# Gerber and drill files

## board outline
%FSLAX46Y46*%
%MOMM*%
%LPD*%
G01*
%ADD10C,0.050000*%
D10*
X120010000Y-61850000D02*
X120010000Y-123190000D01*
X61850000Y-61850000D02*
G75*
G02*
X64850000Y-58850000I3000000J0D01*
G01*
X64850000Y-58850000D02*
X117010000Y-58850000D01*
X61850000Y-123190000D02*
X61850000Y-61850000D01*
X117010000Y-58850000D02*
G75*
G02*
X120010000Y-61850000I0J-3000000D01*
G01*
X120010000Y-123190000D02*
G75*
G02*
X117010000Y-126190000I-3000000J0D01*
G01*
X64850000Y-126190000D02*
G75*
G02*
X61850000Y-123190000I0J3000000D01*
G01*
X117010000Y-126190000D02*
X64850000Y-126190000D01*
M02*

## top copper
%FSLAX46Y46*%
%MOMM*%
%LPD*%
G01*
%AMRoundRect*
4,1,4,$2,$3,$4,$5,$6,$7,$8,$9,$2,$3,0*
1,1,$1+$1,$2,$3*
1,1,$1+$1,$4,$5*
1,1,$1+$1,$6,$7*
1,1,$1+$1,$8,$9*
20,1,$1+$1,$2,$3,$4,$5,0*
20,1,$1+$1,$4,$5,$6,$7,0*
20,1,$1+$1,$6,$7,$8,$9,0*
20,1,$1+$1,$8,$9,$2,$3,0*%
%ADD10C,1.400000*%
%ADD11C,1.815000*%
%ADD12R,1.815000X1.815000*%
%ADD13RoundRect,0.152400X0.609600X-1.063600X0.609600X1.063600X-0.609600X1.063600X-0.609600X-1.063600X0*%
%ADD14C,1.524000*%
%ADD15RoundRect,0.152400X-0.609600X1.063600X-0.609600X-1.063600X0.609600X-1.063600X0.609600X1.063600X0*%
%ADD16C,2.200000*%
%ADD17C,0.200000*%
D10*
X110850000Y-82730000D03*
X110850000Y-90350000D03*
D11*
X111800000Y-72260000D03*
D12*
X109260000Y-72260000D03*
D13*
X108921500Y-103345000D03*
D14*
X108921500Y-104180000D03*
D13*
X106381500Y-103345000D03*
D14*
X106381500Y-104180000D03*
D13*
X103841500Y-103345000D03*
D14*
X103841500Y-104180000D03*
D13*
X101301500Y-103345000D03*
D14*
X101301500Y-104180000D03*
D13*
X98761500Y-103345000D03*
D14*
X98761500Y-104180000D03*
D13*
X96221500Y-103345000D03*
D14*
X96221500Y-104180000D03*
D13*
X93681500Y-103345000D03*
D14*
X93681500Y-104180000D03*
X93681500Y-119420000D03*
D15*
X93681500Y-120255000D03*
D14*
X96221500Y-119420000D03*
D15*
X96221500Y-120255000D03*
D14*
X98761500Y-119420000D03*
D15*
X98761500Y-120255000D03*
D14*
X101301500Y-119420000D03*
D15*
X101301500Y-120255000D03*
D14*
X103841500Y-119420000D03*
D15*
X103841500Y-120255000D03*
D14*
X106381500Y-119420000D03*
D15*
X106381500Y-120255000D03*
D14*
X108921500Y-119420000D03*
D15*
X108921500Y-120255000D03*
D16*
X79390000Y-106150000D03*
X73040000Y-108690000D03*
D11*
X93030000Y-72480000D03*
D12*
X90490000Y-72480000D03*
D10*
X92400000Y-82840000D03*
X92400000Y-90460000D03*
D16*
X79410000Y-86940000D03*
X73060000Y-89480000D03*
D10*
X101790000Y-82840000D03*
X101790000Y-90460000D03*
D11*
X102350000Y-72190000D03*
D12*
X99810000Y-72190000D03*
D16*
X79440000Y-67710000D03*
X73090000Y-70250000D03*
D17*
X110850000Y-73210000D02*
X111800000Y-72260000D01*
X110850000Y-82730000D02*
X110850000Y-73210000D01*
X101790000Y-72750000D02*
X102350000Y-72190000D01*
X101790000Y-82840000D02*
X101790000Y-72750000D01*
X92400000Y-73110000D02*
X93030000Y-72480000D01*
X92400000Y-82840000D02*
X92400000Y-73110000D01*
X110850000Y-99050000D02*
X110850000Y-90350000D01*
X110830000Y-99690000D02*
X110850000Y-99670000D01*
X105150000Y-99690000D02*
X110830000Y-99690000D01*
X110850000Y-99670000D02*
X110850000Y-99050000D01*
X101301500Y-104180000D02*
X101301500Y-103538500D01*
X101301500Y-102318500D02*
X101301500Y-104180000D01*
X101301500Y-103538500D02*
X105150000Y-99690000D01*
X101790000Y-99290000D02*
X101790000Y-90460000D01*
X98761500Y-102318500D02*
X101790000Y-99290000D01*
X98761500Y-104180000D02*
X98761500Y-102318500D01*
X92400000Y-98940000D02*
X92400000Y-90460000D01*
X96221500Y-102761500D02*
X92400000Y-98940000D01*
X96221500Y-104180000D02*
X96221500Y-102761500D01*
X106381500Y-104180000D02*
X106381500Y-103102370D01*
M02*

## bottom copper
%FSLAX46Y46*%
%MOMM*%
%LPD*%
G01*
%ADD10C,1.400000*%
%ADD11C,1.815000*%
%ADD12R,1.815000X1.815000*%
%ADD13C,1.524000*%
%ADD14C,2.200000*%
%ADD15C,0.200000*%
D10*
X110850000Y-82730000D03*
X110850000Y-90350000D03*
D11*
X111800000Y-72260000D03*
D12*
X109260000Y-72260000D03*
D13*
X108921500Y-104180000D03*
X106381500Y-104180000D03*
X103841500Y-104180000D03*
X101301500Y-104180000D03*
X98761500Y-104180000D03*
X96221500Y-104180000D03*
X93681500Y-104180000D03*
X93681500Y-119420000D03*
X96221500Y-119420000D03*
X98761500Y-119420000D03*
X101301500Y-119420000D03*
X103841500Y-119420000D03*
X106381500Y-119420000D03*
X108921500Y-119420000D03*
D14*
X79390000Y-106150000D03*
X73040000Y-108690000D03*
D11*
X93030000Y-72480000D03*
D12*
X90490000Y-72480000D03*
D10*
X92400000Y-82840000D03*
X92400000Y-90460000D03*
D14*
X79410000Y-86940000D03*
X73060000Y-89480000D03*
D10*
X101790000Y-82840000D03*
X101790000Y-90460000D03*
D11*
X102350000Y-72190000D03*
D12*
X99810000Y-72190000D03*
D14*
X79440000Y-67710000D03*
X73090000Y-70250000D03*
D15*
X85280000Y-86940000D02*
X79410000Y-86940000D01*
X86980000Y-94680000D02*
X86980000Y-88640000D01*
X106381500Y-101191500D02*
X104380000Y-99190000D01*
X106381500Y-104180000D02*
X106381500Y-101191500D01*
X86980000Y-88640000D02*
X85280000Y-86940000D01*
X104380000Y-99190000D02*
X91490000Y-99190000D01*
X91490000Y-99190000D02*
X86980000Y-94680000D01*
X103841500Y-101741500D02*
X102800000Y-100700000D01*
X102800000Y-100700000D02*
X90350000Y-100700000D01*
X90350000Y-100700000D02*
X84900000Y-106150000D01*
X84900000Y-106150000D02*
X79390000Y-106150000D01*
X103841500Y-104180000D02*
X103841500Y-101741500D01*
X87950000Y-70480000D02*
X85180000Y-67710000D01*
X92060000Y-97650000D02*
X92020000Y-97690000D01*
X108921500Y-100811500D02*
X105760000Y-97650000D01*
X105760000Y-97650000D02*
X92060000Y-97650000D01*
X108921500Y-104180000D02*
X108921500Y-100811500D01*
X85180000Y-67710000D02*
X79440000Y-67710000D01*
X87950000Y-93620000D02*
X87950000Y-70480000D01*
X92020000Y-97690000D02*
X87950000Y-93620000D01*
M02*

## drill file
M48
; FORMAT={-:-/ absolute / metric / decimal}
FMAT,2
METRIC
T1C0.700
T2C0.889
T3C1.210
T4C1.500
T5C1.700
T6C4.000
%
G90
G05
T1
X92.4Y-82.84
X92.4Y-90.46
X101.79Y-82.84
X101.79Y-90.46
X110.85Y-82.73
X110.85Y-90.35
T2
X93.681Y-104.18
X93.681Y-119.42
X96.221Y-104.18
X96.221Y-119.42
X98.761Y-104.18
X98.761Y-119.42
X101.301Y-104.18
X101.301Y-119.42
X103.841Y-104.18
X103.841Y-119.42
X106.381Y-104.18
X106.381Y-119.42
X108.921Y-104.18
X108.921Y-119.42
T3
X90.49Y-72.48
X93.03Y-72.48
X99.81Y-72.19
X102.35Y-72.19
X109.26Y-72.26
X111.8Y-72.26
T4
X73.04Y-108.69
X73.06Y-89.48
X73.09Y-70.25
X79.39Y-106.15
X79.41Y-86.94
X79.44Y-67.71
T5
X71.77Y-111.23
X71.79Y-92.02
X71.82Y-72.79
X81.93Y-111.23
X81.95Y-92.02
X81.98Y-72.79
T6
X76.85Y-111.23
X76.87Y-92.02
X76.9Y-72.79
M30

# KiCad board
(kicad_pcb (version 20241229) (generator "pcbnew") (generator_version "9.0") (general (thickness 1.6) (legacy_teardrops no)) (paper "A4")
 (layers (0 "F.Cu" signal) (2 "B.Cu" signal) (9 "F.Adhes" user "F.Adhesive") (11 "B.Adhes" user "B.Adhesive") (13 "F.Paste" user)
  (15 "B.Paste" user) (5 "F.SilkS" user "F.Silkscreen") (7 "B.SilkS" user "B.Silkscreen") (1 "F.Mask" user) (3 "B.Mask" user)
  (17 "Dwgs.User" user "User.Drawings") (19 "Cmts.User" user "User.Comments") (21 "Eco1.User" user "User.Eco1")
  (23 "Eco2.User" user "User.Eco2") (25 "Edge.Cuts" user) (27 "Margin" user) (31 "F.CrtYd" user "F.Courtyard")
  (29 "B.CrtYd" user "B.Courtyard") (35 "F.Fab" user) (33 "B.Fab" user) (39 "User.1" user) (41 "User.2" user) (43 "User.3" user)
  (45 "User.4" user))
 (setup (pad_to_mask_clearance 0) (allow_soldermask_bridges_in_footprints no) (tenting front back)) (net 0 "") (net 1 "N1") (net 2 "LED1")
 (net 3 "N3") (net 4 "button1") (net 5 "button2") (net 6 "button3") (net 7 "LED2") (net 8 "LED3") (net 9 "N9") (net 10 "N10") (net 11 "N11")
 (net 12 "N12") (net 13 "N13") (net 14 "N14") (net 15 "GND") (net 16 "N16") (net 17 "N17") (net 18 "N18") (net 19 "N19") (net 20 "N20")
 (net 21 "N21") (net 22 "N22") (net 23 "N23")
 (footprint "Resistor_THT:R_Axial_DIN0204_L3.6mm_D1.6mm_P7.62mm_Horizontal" (layer "F.Cu") (at 110.85 82.73 -90)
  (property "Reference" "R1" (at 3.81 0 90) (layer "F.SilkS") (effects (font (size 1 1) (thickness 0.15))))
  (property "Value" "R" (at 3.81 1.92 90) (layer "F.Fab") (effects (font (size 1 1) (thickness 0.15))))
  (pad "1" thru_hole circle (at 0 0 270) (size 1.4 1.4) (drill 0.7) (layers "*.Cu" "*.Mask") (remove_unused_layers no) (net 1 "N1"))
  (pad "2" thru_hole circle (at 7.62 0 270) (size 1.4 1.4) (drill 0.7) (layers "*.Cu" "*.Mask") (remove_unused_layers no) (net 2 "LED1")))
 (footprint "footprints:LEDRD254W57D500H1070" (layer "F.Cu") (at 110.53 72.26)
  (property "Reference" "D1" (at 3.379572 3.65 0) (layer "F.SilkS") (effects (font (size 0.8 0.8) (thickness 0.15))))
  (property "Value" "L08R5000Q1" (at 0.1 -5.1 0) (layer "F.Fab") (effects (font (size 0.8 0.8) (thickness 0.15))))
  (pad "A" thru_hole circle (at 1.27 0) (size 1.815 1.815) (drill 1.21) (layers "*.Cu" "*.Mask") (remove_unused_layers no) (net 1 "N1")
   (solder_mask_margin 0.102))
  (pad "C" thru_hole rect (at -1.27 0) (size 1.815 1.815) (drill 1.21) (layers "*.Cu" "*.Mask") (remove_unused_layers no) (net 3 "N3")
   (solder_mask_margin 0.102)))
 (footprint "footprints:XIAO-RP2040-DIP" (layer "F.Cu") (at 101.3015 111.8 -90)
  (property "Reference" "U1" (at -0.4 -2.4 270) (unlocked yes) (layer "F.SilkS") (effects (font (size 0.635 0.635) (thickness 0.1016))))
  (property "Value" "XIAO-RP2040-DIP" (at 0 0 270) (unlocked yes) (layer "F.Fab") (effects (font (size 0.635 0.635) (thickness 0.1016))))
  (pad "1" smd roundrect (at -8.455 -7.62 90) (size 2.432 1.524) (layers "F.Cu" "F.Mask") (roundrect_rratio 0.1) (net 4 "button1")
   (thermal_bridge_angle 45))
  (pad "1" thru_hole circle (at -7.62 -7.62 90) (size 1.524 1.524) (drill 0.889) (layers "*.Cu" "*.Mask") (remove_unused_layers no)
   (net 4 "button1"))
  (pad "2" smd roundrect (at -8.455 -5.08 90) (size 2.432 1.524) (layers "F.Cu" "F.Mask") (roundrect_rratio 0.1) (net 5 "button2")
   (thermal_bridge_angle 45))
  (pad "2" thru_hole circle (at -7.62 -5.08 90) (size 1.524 1.524) (drill 0.889) (layers "*.Cu" "*.Mask") (remove_unused_layers no)
   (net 5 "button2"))
  (pad "3" smd roundrect (at -8.455 -2.54 90) (size 2.432 1.524) (layers "F.Cu" "F.Mask") (roundrect_rratio 0.1) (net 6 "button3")
   (thermal_bridge_angle 45))
  (pad "3" thru_hole circle (at -7.62 -2.54 90) (size 1.524 1.524) (drill 0.889) (layers "*.Cu" "*.Mask") (remove_unused_layers no)
   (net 6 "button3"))
  (pad "4" smd roundrect (at -8.455 0 90) (size 2.432 1.524) (layers "F.Cu" "F.Mask") (roundrect_rratio 0.1) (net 2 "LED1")
   (thermal_bridge_angle 45))
  (pad "4" thru_hole circle (at -7.62 0 90) (size 1.524 1.524) (drill 0.889) (layers "*.Cu" "*.Mask") (remove_unused_layers no)
   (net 2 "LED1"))
  (pad "5" smd roundrect (at -8.455 2.54 90) (size 2.432 1.524) (layers "F.Cu" "F.Mask") (roundrect_rratio 0.1) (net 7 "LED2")
   (thermal_bridge_angle 45))
  (pad "5" thru_hole circle (at -7.62 2.54 90) (size 1.524 1.524) (drill 0.889) (layers "*.Cu" "*.Mask") (remove_unused_layers no)
   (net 7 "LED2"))
  (pad "6" smd roundrect (at -8.455 5.08 90) (size 2.432 1.524) (layers "F.Cu" "F.Mask") (roundrect_rratio 0.1) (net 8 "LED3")
   (thermal_bridge_angle 45))
  (pad "6" thru_hole circle (at -7.62 5.08 90) (size 1.524 1.524) (drill 0.889) (layers "*.Cu" "*.Mask") (remove_unused_layers no)
   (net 8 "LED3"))
  (pad "7" smd roundrect (at -8.455 7.62 90) (size 2.432 1.524) (layers "F.Cu" "F.Mask") (roundrect_rratio 0.1) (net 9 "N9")
   (thermal_bridge_angle 45))
  (pad "7" thru_hole circle (at -7.62 7.62 90) (size 1.524 1.524) (drill 0.889) (layers "*.Cu" "*.Mask") (remove_unused_layers no)
   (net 9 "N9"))
  (pad "8" thru_hole circle (at 7.62 7.62 270) (size 1.524 1.524) (drill 0.889) (layers "*.Cu" "*.Mask") (remove_unused_layers no)
   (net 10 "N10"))
  (pad "8" smd roundrect (at 8.455 7.62 270) (size 2.432 1.524) (layers "F.Cu" "F.Mask") (roundrect_rratio 0.1) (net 10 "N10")
   (thermal_bridge_angle 45))
  (pad "9" thru_hole circle (at 7.62 5.08 270) (size 1.524 1.524) (drill 0.889) (layers "*.Cu" "*.Mask") (remove_unused_layers no)
   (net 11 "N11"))
  (pad "9" smd roundrect (at 8.455 5.08 270) (size 2.432 1.524) (layers "F.Cu" "F.Mask") (roundrect_rratio 0.1) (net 11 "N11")
   (thermal_bridge_angle 45))
  (pad "10" thru_hole circle (at 7.62 2.54 270) (size 1.524 1.524) (drill 0.889) (layers "*.Cu" "*.Mask") (remove_unused_layers no)
   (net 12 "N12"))
  (pad "10" smd roundrect (at 8.455 2.54 270) (size 2.432 1.524) (layers "F.Cu" "F.Mask") (roundrect_rratio 0.1) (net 12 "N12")
   (thermal_bridge_angle 45))
  (pad "11" thru_hole circle (at 7.62 0 270) (size 1.524 1.524) (drill 0.889) (layers "*.Cu" "*.Mask") (remove_unused_layers no)
   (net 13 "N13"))
  (pad "11" smd roundrect (at 8.455 0 270) (size 2.432 1.524) (layers "F.Cu" "F.Mask") (roundrect_rratio 0.1) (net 13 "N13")
   (thermal_bridge_angle 45))
  (pad "12" thru_hole circle (at 7.62 -2.54 270) (size 1.524 1.524) (drill 0.889) (layers "*.Cu" "*.Mask") (remove_unused_layers no)
   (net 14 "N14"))
  (pad "12" smd roundrect (at 8.455 -2.54 270) (size 2.432 1.524) (layers "F.Cu" "F.Mask") (roundrect_rratio 0.1) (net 14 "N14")
   (thermal_bridge_angle 45))
  (pad "13" thru_hole circle (at 7.62 -5.08 270) (size 1.524 1.524) (drill 0.889) (layers "*.Cu" "*.Mask") (remove_unused_layers no)
   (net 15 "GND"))
  (pad "13" smd roundrect (at 8.455 -5.08 270) (size 2.432 1.524) (layers "F.Cu" "F.Mask") (roundrect_rratio 0.1) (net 15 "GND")
   (thermal_bridge_angle 45))
  (pad "14" thru_hole circle (at 7.62 -7.62 270) (size 1.524 1.524) (drill 0.889) (layers "*.Cu" "*.Mask") (remove_unused_layers no)
   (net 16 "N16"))
  (pad "14" smd roundrect (at 8.455 -7.62 270) (size 2.432 1.524) (layers "F.Cu" "F.Mask") (roundrect_rratio 0.1) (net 16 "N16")
   (thermal_bridge_angle 45)))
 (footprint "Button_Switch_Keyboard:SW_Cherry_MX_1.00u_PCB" (layer "F.Cu") (at 79.39 106.15)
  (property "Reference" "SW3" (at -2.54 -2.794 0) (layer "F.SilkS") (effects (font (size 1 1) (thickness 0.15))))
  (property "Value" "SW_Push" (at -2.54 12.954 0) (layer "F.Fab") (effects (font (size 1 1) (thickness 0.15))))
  (pad "" np_thru_hole circle (at -7.62 5.08) (size 1.7 1.7) (drill 1.7) (layers "*.Cu" "*.Mask"))
  (pad "" np_thru_hole circle (at -2.54 5.08) (size 4 4) (drill 4) (layers "*.Cu" "*.Mask"))
  (pad "" np_thru_hole circle (at 2.54 5.08) (size 1.7 1.7) (drill 1.7) (layers "*.Cu" "*.Mask"))
  (pad "1" thru_hole circle (at 0 0) (size 2.2 2.2) (drill 1.5) (layers "*.Cu" "*.Mask") (remove_unused_layers no) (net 6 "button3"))
  (pad "2" thru_hole circle (at -6.35 2.54) (size 2.2 2.2) (drill 1.5) (layers "*.Cu" "*.Mask") (remove_unused_layers no) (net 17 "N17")))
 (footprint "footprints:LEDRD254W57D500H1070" (layer "F.Cu") (at 91.76 72.48)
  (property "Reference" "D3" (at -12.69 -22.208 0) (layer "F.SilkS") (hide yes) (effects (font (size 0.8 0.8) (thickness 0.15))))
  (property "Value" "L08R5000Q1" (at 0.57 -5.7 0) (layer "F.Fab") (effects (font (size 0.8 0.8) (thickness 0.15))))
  (pad "A" thru_hole circle (at 1.27 0) (size 1.815 1.815) (drill 1.21) (layers "*.Cu" "*.Mask") (remove_unused_layers no) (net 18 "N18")
   (solder_mask_margin 0.102))
  (pad "C" thru_hole rect (at -1.27 0) (size 1.815 1.815) (drill 1.21) (layers "*.Cu" "*.Mask") (remove_unused_layers no) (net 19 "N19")
   (solder_mask_margin 0.102)))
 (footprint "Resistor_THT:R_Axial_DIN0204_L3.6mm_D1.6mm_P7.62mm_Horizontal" (layer "F.Cu") (at 92.4 82.84 -90)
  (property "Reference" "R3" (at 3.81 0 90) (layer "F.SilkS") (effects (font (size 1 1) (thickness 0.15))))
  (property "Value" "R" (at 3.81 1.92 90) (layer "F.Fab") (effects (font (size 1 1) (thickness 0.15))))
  (pad "1" thru_hole circle (at 0 0 270) (size 1.4 1.4) (drill 0.7) (layers "*.Cu" "*.Mask") (remove_unused_layers no) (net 18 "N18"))
  (pad "2" thru_hole circle (at 7.62 0 270) (size 1.4 1.4) (drill 0.7) (layers "*.Cu" "*.Mask") (remove_unused_layers no) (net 8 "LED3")))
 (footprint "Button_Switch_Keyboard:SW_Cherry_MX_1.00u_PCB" (layer "F.Cu") (at 79.41 86.94)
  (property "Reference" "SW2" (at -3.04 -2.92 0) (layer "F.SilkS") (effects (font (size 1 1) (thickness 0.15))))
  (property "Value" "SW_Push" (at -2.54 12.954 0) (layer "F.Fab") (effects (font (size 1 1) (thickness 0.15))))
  (pad "" np_thru_hole circle (at -7.62 5.08) (size 1.7 1.7) (drill 1.7) (layers "*.Cu" "*.Mask"))
  (pad "" np_thru_hole circle (at -2.54 5.08) (size 4 4) (drill 4) (layers "*.Cu" "*.Mask"))
  (pad "" np_thru_hole circle (at 2.54 5.08) (size 1.7 1.7) (drill 1.7) (layers "*.Cu" "*.Mask"))
  (pad "1" thru_hole circle (at 0 0) (size 2.2 2.2) (drill 1.5) (layers "*.Cu" "*.Mask") (remove_unused_layers no) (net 5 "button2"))
  (pad "2" thru_hole circle (at -6.35 2.54) (size 2.2 2.2) (drill 1.5) (layers "*.Cu" "*.Mask") (remove_unused_layers no) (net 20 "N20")))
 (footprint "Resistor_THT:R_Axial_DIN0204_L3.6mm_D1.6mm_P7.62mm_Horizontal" (layer "F.Cu") (at 101.79 82.84 -90)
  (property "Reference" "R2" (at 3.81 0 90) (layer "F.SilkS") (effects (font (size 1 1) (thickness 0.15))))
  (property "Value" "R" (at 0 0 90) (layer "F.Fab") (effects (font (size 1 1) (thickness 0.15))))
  (pad "1" thru_hole circle (at 0 0 270) (size 1.4 1.4) (drill 0.7) (layers "*.Cu" "*.Mask") (remove_unused_layers no) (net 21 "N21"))
  (pad "2" thru_hole circle (at 7.62 0 270) (size 1.4 1.4) (drill 0.7) (layers "*.Cu" "*.Mask") (remove_unused_layers no) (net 7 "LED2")))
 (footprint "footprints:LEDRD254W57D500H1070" (layer "F.Cu") (at 101.08 72.19)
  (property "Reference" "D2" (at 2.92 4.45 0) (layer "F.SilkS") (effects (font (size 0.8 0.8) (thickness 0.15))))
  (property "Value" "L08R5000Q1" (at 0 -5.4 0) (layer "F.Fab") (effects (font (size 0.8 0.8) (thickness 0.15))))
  (pad "A" thru_hole circle (at 1.27 0) (size 1.815 1.815) (drill 1.21) (layers "*.Cu" "*.Mask") (remove_unused_layers no) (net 21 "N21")
   (solder_mask_margin 0.102))
  (pad "C" thru_hole rect (at -1.27 0) (size 1.815 1.815) (drill 1.21) (layers "*.Cu" "*.Mask") (remove_unused_layers no) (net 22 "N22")
   (solder_mask_margin 0.102)))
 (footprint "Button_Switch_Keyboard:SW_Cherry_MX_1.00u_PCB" (layer "F.Cu") (at 79.44 67.71)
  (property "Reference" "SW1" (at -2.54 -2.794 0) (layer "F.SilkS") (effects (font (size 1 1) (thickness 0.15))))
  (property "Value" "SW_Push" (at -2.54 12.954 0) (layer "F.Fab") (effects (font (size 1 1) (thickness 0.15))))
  (pad "" np_thru_hole circle (at -7.62 5.08) (size 1.7 1.7) (drill 1.7) (layers "*.Cu" "*.Mask"))
  (pad "" np_thru_hole circle (at -2.54 5.08) (size 4 4) (drill 4) (layers "*.Cu" "*.Mask"))
  (pad "" np_thru_hole circle (at 2.54 5.08) (size 1.7 1.7) (drill 1.7) (layers "*.Cu" "*.Mask"))
  (pad "1" thru_hole circle (at 0 0) (size 2.2 2.2) (drill 1.5) (layers "*.Cu" "*.Mask") (remove_unused_layers no) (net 4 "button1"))
  (pad "2" thru_hole circle (at -6.35 2.54) (size 2.2 2.2) (drill 1.5) (layers "*.Cu" "*.Mask") (remove_unused_layers no) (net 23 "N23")))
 (gr_line (start 120.01 61.85) (end 120.01 123.19) (stroke (width 0.05) (type default)) (layer "Edge.Cuts"))
 (gr_arc (start 61.85 61.85) (mid 62.72868 59.72868) (end 64.85 58.85) (stroke (width 0.05) (type default)) (layer "Edge.Cuts"))
 (gr_line (start 64.85 58.85) (end 117.01 58.85) (stroke (width 0.05) (type default)) (layer "Edge.Cuts"))
 (gr_line (start 61.85 123.19) (end 61.85 61.85) (stroke (width 0.05) (type default)) (layer "Edge.Cuts"))
 (gr_arc (start 117.01 58.85) (mid 119.13132 59.72868) (end 120.01 61.85) (stroke (width 0.05) (type default)) (layer "Edge.Cuts"))
 (gr_arc (start 120.01 123.19) (mid 119.13132 125.31132) (end 117.01 126.19) (stroke (width 0.05) (type default)) (layer "Edge.Cuts"))
 (gr_arc (start 64.85 126.19) (mid 62.72868 125.31132) (end 61.85 123.19) (stroke (width 0.05) (type default)) (layer "Edge.Cuts"))
 (gr_line (start 117.01 126.19) (end 64.85 126.19) (stroke (width 0.05) (type default)) (layer "Edge.Cuts"))
 (segment (start 110.85 73.21) (end 111.8 72.26) (width 0.2) (layer "F.Cu") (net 1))
 (segment (start 110.85 82.73) (end 110.85 73.21) (width 0.2) (layer "F.Cu") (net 1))
 (segment (start 101.79 72.75) (end 102.35 72.19) (width 0.2) (layer "F.Cu") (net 21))
 (segment (start 101.79 82.84) (end 101.79 72.75) (width 0.2) (layer "F.Cu") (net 21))
 (segment (start 92.4 73.11) (end 93.03 72.48) (width 0.2) (layer "F.Cu") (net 18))
 (segment (start 92.4 82.84) (end 92.4 73.11) (width 0.2) (layer "F.Cu") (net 18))
 (segment (start 110.85 99.05) (end 110.85 90.35) (width 0.2) (layer "F.Cu") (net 2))
 (segment (start 110.83 99.69) (end 110.85 99.67) (width 0.2) (layer "F.Cu") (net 2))
 (segment (start 105.15 99.69) (end 110.83 99.69) (width 0.2) (layer "F.Cu") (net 2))
 (segment (start 110.85 99.67) (end 110.85 99.05) (width 0.2) (layer "F.Cu") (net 2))
 (segment (start 101.3015 104.18) (end 101.3015 103.5385) (width 0.2) (layer "F.Cu") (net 2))
 (segment (start 101.3015 102.3185) (end 101.3015 104.18) (width 0.2) (layer "F.Cu") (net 2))
 (segment (start 101.3015 103.5385) (end 105.15 99.69) (width 0.2) (layer "F.Cu") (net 2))
 (segment (start 101.79 99.29) (end 101.79 90.46) (width 0.2) (layer "F.Cu") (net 7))
 (segment (start 98.7615 102.3185) (end 101.79 99.29) (width 0.2) (layer "F.Cu") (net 7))
 (segment (start 98.7615 104.18) (end 98.7615 102.3185) (width 0.2) (layer "F.Cu") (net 7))
 (segment (start 92.4 98.94) (end 92.4 90.46) (width 0.2) (layer "F.Cu") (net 8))
 (segment (start 96.2215 102.7615) (end 92.4 98.94) (width 0.2) (layer "F.Cu") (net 8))
 (segment (start 96.2215 104.18) (end 96.2215 102.7615) (width 0.2) (layer "F.Cu") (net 8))
 (segment (start 106.3815 104.18) (end 106.3815 103.10237) (width 0.2) (layer "F.Cu") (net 5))
 (segment (start 85.28 86.94) (end 79.41 86.94) (width 0.2) (layer "B.Cu") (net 5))
 (segment (start 86.98 94.68) (end 86.98 88.64) (width 0.2) (layer "B.Cu") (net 5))
 (segment (start 106.3815 101.1915) (end 104.38 99.19) (width 0.2) (layer "B.Cu") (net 5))
 (segment (start 106.3815 104.18) (end 106.3815 101.1915) (width 0.2) (layer "B.Cu") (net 5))
 (segment (start 86.98 88.64) (end 85.28 86.94) (width 0.2) (layer "B.Cu") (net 5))
 (segment (start 104.38 99.19) (end 91.49 99.19) (width 0.2) (layer "B.Cu") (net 5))
 (segment (start 91.49 99.19) (end 86.98 94.68) (width 0.2) (layer "B.Cu") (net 5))
 (segment (start 103.8415 101.7415) (end 102.8 100.7) (width 0.2) (layer "B.Cu") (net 6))
 (segment (start 102.8 100.7) (end 90.35 100.7) (width 0.2) (layer "B.Cu") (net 6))
 (segment (start 90.35 100.7) (end 84.9 106.15) (width 0.2) (layer "B.Cu") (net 6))
 (segment (start 84.9 106.15) (end 79.39 106.15) (width 0.2) (layer "B.Cu") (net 6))
 (segment (start 103.8415 104.18) (end 103.8415 101.7415) (width 0.2) (layer "B.Cu") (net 6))
 (segment (start 87.95 70.48) (end 85.18 67.71) (width 0.2) (layer "B.Cu") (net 4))
 (segment (start 92.06 97.65) (end 92.02 97.69) (width 0.2) (layer "B.Cu") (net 4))
 (segment (start 108.9215 100.8115) (end 105.76 97.65) (width 0.2) (layer "B.Cu") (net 4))
 (segment (start 105.76 97.65) (end 92.06 97.65) (width 0.2) (layer "B.Cu") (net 4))
 (segment (start 108.9215 104.18) (end 108.9215 100.8115) (width 0.2) (layer "B.Cu") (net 4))
 (segment (start 85.18 67.71) (end 79.44 67.71) (width 0.2) (layer "B.Cu") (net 4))
 (segment (start 87.95 93.62) (end 87.95 70.48) (width 0.2) (layer "B.Cu") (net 4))
 (segment (start 92.02 97.69) (end 87.95 93.62) (width 0.2) (layer "B.Cu") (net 4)))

